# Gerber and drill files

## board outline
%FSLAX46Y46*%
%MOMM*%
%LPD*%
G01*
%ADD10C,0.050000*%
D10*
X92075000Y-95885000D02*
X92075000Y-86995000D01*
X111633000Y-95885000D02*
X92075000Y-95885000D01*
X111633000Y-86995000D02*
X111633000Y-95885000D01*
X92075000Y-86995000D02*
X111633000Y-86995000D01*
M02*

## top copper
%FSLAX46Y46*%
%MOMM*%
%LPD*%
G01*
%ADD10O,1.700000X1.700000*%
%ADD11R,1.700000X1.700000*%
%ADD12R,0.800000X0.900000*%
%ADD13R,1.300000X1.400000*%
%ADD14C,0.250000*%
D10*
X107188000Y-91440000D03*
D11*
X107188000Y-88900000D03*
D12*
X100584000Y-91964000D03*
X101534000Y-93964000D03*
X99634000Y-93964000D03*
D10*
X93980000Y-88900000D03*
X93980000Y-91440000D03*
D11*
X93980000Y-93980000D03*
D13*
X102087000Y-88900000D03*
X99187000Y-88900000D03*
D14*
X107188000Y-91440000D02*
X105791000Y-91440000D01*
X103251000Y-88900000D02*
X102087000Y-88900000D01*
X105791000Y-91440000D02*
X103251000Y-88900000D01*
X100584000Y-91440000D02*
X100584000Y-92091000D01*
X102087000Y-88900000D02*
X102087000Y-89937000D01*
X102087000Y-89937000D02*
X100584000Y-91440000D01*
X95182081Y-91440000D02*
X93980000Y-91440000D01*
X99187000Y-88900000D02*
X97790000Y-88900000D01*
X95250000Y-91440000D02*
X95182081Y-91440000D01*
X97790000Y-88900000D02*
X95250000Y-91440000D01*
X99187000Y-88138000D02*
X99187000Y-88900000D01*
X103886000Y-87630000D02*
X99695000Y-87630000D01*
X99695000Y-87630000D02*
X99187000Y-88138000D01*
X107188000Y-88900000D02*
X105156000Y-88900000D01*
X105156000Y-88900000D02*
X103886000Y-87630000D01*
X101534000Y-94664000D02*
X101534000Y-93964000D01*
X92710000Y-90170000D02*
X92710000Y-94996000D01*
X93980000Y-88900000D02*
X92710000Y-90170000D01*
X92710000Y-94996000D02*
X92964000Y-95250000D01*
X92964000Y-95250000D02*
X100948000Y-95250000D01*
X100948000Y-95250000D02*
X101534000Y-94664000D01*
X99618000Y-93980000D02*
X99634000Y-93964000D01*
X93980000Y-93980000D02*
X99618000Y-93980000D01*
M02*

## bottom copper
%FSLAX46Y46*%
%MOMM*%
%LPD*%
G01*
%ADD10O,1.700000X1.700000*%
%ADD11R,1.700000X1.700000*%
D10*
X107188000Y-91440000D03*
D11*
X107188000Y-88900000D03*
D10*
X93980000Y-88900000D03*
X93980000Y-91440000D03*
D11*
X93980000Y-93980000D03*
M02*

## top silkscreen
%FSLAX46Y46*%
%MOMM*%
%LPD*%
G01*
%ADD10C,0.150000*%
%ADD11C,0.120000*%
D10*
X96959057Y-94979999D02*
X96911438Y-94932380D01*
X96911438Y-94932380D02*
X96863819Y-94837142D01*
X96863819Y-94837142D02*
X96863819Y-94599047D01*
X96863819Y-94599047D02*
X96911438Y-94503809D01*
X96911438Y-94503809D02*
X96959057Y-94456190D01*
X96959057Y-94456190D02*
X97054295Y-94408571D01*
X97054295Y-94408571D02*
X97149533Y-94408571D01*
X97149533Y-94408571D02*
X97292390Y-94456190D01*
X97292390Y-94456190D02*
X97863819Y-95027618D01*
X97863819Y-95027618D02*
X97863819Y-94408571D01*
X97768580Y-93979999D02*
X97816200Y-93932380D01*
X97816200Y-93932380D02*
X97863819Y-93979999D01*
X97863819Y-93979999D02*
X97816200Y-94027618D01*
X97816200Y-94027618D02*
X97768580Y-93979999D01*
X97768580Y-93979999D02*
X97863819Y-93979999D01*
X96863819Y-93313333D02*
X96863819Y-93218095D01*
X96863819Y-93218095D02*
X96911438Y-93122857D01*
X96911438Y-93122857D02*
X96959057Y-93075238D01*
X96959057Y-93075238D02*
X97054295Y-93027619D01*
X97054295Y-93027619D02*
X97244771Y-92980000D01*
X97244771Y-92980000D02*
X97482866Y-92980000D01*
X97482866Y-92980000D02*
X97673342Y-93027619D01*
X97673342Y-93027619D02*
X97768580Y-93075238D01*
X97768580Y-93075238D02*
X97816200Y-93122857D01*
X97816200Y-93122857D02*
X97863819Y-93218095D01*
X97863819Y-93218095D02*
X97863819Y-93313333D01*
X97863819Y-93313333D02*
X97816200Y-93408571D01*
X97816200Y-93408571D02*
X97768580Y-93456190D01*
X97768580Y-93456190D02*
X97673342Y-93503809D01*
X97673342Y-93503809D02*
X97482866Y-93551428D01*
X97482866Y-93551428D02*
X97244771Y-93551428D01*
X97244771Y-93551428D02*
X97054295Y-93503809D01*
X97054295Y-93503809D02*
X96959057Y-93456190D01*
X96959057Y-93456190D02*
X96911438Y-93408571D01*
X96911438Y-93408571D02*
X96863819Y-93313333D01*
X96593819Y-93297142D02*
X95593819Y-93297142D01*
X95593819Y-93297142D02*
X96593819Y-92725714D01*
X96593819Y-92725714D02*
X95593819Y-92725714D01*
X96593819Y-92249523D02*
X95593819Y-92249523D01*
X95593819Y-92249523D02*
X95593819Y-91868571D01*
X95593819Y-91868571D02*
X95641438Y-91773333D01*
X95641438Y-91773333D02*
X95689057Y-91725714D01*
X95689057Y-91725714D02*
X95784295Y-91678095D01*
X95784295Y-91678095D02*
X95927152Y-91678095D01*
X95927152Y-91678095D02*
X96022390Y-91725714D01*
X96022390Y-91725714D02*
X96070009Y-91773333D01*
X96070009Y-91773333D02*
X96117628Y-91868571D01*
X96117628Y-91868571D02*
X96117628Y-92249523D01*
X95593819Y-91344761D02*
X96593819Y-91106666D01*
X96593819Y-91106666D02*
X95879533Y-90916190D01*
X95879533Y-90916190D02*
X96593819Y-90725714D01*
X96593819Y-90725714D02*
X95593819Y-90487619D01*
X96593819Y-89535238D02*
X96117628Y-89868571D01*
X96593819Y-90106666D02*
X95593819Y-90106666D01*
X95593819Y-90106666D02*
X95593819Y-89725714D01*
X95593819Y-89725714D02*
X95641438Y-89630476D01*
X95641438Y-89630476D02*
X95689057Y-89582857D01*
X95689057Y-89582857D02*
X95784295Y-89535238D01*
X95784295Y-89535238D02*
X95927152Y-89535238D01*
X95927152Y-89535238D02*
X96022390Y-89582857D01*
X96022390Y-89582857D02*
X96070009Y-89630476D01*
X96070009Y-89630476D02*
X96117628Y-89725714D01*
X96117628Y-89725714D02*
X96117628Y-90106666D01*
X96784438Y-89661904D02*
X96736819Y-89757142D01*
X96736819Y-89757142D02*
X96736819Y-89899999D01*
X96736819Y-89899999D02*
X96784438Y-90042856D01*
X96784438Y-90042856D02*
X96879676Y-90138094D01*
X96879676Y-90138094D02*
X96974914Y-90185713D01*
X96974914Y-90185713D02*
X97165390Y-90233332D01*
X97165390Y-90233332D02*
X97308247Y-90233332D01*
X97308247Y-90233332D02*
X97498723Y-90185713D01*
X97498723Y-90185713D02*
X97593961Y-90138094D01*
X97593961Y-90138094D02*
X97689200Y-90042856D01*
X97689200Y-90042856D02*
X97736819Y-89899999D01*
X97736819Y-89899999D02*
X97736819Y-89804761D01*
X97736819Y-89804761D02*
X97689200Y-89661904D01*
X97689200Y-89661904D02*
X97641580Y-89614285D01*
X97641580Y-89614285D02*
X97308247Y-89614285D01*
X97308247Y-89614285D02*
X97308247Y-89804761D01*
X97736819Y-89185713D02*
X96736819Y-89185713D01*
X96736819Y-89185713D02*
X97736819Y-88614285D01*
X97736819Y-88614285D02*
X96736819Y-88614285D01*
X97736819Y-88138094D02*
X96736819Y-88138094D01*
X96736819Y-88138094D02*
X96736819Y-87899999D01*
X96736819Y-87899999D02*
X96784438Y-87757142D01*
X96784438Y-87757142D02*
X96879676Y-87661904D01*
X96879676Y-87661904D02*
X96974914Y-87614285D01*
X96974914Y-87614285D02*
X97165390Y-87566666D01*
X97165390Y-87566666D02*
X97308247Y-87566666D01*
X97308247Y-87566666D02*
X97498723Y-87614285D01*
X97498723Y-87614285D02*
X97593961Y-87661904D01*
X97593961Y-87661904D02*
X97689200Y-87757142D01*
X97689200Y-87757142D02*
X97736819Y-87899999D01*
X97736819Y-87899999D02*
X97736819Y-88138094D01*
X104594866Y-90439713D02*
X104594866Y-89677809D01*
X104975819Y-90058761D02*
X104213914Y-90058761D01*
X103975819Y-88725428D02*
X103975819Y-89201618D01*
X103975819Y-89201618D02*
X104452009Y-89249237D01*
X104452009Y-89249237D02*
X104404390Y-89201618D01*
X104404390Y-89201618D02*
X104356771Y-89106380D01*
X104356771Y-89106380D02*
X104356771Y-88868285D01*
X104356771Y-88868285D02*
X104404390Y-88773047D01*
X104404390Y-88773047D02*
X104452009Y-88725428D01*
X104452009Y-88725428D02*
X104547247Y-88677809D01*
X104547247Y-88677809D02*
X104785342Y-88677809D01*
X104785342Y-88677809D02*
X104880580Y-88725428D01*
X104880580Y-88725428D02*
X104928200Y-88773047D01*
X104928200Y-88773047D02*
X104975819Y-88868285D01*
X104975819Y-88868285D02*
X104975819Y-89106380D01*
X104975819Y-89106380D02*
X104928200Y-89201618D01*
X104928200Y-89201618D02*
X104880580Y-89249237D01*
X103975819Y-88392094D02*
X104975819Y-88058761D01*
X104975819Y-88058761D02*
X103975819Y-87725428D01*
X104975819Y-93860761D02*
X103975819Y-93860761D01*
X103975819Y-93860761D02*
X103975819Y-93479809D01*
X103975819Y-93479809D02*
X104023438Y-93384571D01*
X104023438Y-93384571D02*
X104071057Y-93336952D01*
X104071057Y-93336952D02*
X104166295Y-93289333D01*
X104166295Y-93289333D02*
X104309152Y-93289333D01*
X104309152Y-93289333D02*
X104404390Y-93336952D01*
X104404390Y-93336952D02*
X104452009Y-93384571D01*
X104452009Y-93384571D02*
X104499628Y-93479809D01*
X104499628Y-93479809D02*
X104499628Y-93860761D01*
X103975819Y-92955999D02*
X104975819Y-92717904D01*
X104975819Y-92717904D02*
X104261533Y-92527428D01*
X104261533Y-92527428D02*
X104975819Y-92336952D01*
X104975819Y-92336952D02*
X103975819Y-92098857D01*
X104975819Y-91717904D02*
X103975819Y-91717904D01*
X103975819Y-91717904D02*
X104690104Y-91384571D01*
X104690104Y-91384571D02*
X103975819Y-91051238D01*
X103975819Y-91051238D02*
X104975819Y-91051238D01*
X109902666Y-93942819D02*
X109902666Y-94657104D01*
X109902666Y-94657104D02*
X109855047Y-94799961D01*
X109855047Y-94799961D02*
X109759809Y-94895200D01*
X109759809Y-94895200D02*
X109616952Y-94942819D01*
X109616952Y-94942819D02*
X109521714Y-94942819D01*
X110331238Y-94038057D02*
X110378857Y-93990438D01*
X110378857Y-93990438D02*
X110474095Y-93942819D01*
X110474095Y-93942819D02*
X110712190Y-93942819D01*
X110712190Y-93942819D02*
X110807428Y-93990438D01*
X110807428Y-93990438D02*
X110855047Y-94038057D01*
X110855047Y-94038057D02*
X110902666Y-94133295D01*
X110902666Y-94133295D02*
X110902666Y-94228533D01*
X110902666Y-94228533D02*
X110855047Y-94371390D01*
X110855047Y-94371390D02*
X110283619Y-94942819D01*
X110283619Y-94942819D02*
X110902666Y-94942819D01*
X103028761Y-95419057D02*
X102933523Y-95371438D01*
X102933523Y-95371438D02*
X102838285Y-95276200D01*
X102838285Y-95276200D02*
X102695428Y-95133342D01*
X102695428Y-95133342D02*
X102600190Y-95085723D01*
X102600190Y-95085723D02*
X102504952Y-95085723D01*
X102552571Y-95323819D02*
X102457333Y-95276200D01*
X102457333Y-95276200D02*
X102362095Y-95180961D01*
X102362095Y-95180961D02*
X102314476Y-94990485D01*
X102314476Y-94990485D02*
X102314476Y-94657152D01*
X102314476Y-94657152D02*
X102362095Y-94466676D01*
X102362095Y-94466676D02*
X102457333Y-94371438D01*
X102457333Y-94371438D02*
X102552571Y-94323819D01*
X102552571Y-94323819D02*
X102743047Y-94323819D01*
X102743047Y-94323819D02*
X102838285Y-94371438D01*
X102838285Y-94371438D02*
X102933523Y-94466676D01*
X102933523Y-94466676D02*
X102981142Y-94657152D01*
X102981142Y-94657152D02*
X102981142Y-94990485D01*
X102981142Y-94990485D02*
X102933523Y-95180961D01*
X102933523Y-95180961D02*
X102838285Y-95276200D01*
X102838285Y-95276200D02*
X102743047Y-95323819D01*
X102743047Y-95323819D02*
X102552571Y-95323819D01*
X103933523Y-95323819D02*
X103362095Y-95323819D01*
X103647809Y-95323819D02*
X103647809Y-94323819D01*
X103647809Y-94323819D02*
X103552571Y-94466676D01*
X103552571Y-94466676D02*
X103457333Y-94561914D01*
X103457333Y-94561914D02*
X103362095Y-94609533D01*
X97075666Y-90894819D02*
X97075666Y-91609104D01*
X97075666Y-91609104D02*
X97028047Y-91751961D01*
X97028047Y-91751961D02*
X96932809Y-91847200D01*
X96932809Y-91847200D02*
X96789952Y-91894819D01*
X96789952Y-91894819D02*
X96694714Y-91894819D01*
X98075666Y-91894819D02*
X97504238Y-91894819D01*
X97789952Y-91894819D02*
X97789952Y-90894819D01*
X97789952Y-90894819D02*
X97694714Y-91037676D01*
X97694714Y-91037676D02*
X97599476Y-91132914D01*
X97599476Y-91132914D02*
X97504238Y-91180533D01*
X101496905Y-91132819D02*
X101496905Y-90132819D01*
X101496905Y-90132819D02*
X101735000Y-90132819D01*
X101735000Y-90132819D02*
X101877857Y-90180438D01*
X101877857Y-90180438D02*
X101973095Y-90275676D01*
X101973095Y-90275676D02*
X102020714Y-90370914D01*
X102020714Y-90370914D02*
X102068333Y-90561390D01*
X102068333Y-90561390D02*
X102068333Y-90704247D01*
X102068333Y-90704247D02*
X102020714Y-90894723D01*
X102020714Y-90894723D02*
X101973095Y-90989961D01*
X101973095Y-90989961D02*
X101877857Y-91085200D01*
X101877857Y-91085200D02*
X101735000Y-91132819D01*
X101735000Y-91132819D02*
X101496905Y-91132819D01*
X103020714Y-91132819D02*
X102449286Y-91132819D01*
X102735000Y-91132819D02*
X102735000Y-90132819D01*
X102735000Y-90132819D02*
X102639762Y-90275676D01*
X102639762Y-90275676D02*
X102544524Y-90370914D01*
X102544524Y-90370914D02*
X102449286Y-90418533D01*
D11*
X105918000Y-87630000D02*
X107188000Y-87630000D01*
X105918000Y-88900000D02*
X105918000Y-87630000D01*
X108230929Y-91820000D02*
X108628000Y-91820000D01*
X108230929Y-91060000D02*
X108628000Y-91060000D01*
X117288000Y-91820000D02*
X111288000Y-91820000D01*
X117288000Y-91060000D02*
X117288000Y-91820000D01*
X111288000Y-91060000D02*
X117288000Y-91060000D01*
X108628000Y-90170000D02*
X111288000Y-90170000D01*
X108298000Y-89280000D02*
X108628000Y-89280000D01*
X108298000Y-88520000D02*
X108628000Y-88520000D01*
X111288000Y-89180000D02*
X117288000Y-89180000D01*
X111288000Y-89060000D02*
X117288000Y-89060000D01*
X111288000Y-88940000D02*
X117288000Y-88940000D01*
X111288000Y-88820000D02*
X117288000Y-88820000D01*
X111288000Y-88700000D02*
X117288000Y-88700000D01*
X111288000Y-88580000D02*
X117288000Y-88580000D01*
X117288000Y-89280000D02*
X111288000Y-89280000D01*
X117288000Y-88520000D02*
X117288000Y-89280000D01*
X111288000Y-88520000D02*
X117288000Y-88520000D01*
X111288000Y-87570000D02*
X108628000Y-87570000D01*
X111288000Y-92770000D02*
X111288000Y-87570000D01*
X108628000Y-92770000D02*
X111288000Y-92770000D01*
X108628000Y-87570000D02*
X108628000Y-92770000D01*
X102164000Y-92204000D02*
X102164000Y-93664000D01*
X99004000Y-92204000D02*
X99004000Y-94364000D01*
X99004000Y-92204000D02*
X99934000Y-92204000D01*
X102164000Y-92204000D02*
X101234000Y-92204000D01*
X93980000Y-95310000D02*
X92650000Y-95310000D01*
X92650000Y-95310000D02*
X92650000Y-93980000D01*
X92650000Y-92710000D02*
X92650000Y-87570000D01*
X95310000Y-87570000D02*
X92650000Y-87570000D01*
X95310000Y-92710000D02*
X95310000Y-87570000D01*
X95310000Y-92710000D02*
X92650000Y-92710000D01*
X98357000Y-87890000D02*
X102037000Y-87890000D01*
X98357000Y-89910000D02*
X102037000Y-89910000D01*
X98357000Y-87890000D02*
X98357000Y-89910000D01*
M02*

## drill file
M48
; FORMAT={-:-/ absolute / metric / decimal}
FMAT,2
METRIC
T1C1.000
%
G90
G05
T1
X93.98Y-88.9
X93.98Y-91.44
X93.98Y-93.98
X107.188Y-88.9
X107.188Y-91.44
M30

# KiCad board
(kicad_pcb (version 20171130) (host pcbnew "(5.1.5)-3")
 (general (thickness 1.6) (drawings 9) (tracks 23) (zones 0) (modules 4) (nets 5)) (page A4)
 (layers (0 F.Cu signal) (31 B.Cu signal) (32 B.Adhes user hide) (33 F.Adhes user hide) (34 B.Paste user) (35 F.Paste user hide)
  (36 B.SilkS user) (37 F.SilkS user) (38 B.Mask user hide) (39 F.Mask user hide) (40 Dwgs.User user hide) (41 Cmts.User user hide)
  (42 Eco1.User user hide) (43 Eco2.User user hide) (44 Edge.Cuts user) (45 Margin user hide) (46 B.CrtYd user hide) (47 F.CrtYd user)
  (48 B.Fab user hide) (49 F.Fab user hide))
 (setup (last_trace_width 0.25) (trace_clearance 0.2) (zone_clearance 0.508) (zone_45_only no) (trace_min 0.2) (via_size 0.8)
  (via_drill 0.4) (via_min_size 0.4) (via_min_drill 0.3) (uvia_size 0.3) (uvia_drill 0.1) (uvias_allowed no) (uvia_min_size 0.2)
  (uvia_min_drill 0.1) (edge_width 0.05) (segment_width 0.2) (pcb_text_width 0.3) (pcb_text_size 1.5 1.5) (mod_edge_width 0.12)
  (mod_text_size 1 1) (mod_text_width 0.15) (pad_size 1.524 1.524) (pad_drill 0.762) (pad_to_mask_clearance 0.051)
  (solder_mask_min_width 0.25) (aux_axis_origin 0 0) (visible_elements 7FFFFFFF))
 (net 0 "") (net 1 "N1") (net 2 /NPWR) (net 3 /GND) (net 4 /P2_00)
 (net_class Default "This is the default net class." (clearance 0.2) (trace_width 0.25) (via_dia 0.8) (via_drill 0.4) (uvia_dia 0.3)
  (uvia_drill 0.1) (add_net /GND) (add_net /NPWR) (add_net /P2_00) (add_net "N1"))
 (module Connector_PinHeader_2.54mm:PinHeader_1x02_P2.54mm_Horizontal (layer F.Cu) (at 107.188 88.9)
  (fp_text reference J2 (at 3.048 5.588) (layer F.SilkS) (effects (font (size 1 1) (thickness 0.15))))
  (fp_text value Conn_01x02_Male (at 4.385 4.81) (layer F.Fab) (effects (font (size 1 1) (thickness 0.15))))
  (fp_line (start -1.27 -1.27) (end 0 -1.27) (layer F.SilkS) (width 0.12))
  (fp_line (start -1.27 0) (end -1.27 -1.27) (layer F.SilkS) (width 0.12))
  (fp_line (start 1.042929 2.92) (end 1.44 2.92) (layer F.SilkS) (width 0.12))
  (fp_line (start 1.042929 2.16) (end 1.44 2.16) (layer F.SilkS) (width 0.12))
  (fp_line (start 10.1 2.92) (end 4.1 2.92) (layer F.SilkS) (width 0.12))
  (fp_line (start 10.1 2.16) (end 10.1 2.92) (layer F.SilkS) (width 0.12))
  (fp_line (start 4.1 2.16) (end 10.1 2.16) (layer F.SilkS) (width 0.12))
  (fp_line (start 1.44 1.27) (end 4.1 1.27) (layer F.SilkS) (width 0.12))
  (fp_line (start 1.11 0.38) (end 1.44 0.38) (layer F.SilkS) (width 0.12))
  (fp_line (start 1.11 -0.38) (end 1.44 -0.38) (layer F.SilkS) (width 0.12))
  (fp_line (start 4.1 0.28) (end 10.1 0.28) (layer F.SilkS) (width 0.12))
  (fp_line (start 4.1 0.16) (end 10.1 0.16) (layer F.SilkS) (width 0.12))
  (fp_line (start 4.1 0.04) (end 10.1 0.04) (layer F.SilkS) (width 0.12))
  (fp_line (start 4.1 -0.08) (end 10.1 -0.08) (layer F.SilkS) (width 0.12))
  (fp_line (start 4.1 -0.2) (end 10.1 -0.2) (layer F.SilkS) (width 0.12))
  (fp_line (start 4.1 -0.32) (end 10.1 -0.32) (layer F.SilkS) (width 0.12))
  (fp_line (start 10.1 0.38) (end 4.1 0.38) (layer F.SilkS) (width 0.12))
  (fp_line (start 10.1 -0.38) (end 10.1 0.38) (layer F.SilkS) (width 0.12))
  (fp_line (start 4.1 -0.38) (end 10.1 -0.38) (layer F.SilkS) (width 0.12))
  (fp_line (start 4.1 -1.33) (end 1.44 -1.33) (layer F.SilkS) (width 0.12))
  (fp_line (start 4.1 3.87) (end 4.1 -1.33) (layer F.SilkS) (width 0.12))
  (fp_line (start 1.44 3.87) (end 4.1 3.87) (layer F.SilkS) (width 0.12))
  (fp_line (start 1.44 -1.33) (end 1.44 3.87) (layer F.SilkS) (width 0.12))
  (pad 2 thru_hole oval (at 0 2.54) (size 1.7 1.7) (drill 1) (layers *.Cu *.Mask) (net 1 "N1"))
  (pad 1 thru_hole rect (at 0 0) (size 1.7 1.7) (drill 1) (layers *.Cu *.Mask) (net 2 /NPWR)))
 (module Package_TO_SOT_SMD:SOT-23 (layer F.Cu) (at 100.584 92.964 90)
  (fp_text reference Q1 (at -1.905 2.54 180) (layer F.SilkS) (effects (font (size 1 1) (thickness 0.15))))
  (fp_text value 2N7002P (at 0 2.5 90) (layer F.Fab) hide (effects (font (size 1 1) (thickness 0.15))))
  (fp_line (start 0.76 1.58) (end -0.7 1.58) (layer F.SilkS) (width 0.12))
  (fp_line (start 0.76 -1.58) (end -1.4 -1.58) (layer F.SilkS) (width 0.12))
  (fp_line (start 0.76 -1.58) (end 0.76 -0.65) (layer F.SilkS) (width 0.12))
  (fp_line (start 0.76 1.58) (end 0.76 0.65) (layer F.SilkS) (width 0.12))
  (pad 3 smd rect (at 1 0 90) (size 0.9 0.8) (layers F.Cu F.Paste F.Mask) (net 1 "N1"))
  (pad 2 smd rect (at -1 0.95 90) (size 0.9 0.8) (layers F.Cu F.Paste F.Mask) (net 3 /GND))
  (pad 1 smd rect (at -1 -0.95 90) (size 0.9 0.8) (layers F.Cu F.Paste F.Mask) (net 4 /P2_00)))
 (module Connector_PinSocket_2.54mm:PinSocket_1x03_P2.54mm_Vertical (layer F.Cu) (at 93.98 93.98 180)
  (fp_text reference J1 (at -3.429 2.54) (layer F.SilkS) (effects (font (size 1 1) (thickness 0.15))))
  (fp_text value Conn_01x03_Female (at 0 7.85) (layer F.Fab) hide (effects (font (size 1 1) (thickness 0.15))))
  (fp_line (start 0 -1.33) (end 1.33 -1.33) (layer F.SilkS) (width 0.12))
  (fp_line (start 1.33 -1.33) (end 1.33 0) (layer F.SilkS) (width 0.12))
  (fp_line (start 1.33 1.27) (end 1.33 6.41) (layer F.SilkS) (width 0.12))
  (fp_line (start -1.33 6.41) (end 1.33 6.41) (layer F.SilkS) (width 0.12))
  (fp_line (start -1.33 1.27) (end -1.33 6.41) (layer F.SilkS) (width 0.12))
  (fp_line (start -1.33 1.27) (end 1.33 1.27) (layer F.SilkS) (width 0.12))
  (pad 3 thru_hole oval (at 0 5.08 180) (size 1.7 1.7) (drill 1) (layers *.Cu *.Mask) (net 3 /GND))
  (pad 2 thru_hole oval (at 0 2.54 180) (size 1.7 1.7) (drill 1) (layers *.Cu *.Mask) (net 2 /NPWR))
  (pad 1 thru_hole rect (at 0 0 180) (size 1.7 1.7) (drill 1) (layers *.Cu *.Mask) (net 4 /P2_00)))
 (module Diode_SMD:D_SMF (layer F.Cu) (at 100.637 88.9)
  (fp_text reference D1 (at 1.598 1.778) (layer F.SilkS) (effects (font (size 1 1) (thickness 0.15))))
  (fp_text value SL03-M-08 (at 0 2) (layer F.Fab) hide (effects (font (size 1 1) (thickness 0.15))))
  (fp_line (start -2.28 -1.01) (end 1.4 -1.01) (layer F.SilkS) (width 0.12))
  (fp_line (start -2.28 1.01) (end 1.4 1.01) (layer F.SilkS) (width 0.12))
  (fp_line (start -2.28 -1.01) (end -2.28 1.01) (layer F.SilkS) (width 0.12))
  (pad 2 smd rect (at 1.45 0) (size 1.3 1.4) (layers F.Cu F.Paste F.Mask) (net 1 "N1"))
  (pad 1 smd rect (at -1.45 0) (size 1.3 1.4) (layers F.Cu F.Paste F.Mask) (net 2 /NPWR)))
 (gr_line (start 92.075 95.885) (end 92.075 86.995) (layer Edge.Cuts) (width 0.05))
 (gr_line (start 111.633 95.885) (end 92.075 95.885) (layer Edge.Cuts) (width 0.05))
 (gr_line (start 111.633 86.995) (end 111.633 95.885) (layer Edge.Cuts) (width 0.05))
 (gr_line (start 92.075 86.995) (end 111.633 86.995) (layer Edge.Cuts) (width 0.05))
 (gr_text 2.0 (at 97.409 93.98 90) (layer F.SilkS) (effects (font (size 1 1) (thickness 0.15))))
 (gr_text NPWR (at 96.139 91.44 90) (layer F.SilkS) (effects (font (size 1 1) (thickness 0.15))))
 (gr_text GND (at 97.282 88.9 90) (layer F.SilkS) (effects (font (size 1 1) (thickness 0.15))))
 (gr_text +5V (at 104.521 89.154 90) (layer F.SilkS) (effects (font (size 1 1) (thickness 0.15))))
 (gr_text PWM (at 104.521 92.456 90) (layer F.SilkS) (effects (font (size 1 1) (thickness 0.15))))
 (segment (start 107.188 91.44) (end 105.791 91.44) (width 0.25) (layer F.Cu) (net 1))
 (segment (start 103.251 88.9) (end 102.087 88.9) (width 0.25) (layer F.Cu) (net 1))
 (segment (start 105.791 91.44) (end 103.251 88.9) (width 0.25) (layer F.Cu) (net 1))
 (segment (start 100.584 91.44) (end 100.584 92.091) (width 0.25) (layer F.Cu) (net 1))
 (segment (start 102.087 88.9) (end 102.087 89.937) (width 0.25) (layer F.Cu) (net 1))
 (segment (start 102.087 89.937) (end 100.584 91.44) (width 0.25) (layer F.Cu) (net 1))
 (segment (start 95.182081 91.44) (end 93.98 91.44) (width 0.25) (layer F.Cu) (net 2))
 (segment (start 99.187 88.9) (end 97.79 88.9) (width 0.25) (layer F.Cu) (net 2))
 (segment (start 95.25 91.44) (end 95.182081 91.44) (width 0.25) (layer F.Cu) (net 2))
 (segment (start 97.79 88.9) (end 95.25 91.44) (width 0.25) (layer F.Cu) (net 2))
 (segment (start 99.187 88.138) (end 99.187 88.9) (width 0.25) (layer F.Cu) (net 2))
 (segment (start 103.886 87.63) (end 99.695 87.63) (width 0.25) (layer F.Cu) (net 2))
 (segment (start 99.695 87.63) (end 99.187 88.138) (width 0.25) (layer F.Cu) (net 2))
 (segment (start 107.188 88.9) (end 105.156 88.9) (width 0.25) (layer F.Cu) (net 2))
 (segment (start 105.156 88.9) (end 103.886 87.63) (width 0.25) (layer F.Cu) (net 2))
 (segment (start 101.534 94.664) (end 101.534 93.964) (width 0.25) (layer F.Cu) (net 3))
 (segment (start 92.71 90.17) (end 92.71 94.996) (width 0.25) (layer F.Cu) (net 3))
 (segment (start 93.98 88.9) (end 92.71 90.17) (width 0.25) (layer F.Cu) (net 3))
 (segment (start 92.71 94.996) (end 92.964 95.25) (width 0.25) (layer F.Cu) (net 3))
 (segment (start 92.964 95.25) (end 100.948 95.25) (width 0.25) (layer F.Cu) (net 3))
 (segment (start 100.948 95.25) (end 101.534 94.664) (width 0.25) (layer F.Cu) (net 3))
 (segment (start 99.618 93.98) (end 99.634 93.964) (width 0.25) (layer F.Cu) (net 4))
 (segment (start 93.98 93.98) (end 99.618 93.98) (width 0.25) (layer F.Cu) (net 4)))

